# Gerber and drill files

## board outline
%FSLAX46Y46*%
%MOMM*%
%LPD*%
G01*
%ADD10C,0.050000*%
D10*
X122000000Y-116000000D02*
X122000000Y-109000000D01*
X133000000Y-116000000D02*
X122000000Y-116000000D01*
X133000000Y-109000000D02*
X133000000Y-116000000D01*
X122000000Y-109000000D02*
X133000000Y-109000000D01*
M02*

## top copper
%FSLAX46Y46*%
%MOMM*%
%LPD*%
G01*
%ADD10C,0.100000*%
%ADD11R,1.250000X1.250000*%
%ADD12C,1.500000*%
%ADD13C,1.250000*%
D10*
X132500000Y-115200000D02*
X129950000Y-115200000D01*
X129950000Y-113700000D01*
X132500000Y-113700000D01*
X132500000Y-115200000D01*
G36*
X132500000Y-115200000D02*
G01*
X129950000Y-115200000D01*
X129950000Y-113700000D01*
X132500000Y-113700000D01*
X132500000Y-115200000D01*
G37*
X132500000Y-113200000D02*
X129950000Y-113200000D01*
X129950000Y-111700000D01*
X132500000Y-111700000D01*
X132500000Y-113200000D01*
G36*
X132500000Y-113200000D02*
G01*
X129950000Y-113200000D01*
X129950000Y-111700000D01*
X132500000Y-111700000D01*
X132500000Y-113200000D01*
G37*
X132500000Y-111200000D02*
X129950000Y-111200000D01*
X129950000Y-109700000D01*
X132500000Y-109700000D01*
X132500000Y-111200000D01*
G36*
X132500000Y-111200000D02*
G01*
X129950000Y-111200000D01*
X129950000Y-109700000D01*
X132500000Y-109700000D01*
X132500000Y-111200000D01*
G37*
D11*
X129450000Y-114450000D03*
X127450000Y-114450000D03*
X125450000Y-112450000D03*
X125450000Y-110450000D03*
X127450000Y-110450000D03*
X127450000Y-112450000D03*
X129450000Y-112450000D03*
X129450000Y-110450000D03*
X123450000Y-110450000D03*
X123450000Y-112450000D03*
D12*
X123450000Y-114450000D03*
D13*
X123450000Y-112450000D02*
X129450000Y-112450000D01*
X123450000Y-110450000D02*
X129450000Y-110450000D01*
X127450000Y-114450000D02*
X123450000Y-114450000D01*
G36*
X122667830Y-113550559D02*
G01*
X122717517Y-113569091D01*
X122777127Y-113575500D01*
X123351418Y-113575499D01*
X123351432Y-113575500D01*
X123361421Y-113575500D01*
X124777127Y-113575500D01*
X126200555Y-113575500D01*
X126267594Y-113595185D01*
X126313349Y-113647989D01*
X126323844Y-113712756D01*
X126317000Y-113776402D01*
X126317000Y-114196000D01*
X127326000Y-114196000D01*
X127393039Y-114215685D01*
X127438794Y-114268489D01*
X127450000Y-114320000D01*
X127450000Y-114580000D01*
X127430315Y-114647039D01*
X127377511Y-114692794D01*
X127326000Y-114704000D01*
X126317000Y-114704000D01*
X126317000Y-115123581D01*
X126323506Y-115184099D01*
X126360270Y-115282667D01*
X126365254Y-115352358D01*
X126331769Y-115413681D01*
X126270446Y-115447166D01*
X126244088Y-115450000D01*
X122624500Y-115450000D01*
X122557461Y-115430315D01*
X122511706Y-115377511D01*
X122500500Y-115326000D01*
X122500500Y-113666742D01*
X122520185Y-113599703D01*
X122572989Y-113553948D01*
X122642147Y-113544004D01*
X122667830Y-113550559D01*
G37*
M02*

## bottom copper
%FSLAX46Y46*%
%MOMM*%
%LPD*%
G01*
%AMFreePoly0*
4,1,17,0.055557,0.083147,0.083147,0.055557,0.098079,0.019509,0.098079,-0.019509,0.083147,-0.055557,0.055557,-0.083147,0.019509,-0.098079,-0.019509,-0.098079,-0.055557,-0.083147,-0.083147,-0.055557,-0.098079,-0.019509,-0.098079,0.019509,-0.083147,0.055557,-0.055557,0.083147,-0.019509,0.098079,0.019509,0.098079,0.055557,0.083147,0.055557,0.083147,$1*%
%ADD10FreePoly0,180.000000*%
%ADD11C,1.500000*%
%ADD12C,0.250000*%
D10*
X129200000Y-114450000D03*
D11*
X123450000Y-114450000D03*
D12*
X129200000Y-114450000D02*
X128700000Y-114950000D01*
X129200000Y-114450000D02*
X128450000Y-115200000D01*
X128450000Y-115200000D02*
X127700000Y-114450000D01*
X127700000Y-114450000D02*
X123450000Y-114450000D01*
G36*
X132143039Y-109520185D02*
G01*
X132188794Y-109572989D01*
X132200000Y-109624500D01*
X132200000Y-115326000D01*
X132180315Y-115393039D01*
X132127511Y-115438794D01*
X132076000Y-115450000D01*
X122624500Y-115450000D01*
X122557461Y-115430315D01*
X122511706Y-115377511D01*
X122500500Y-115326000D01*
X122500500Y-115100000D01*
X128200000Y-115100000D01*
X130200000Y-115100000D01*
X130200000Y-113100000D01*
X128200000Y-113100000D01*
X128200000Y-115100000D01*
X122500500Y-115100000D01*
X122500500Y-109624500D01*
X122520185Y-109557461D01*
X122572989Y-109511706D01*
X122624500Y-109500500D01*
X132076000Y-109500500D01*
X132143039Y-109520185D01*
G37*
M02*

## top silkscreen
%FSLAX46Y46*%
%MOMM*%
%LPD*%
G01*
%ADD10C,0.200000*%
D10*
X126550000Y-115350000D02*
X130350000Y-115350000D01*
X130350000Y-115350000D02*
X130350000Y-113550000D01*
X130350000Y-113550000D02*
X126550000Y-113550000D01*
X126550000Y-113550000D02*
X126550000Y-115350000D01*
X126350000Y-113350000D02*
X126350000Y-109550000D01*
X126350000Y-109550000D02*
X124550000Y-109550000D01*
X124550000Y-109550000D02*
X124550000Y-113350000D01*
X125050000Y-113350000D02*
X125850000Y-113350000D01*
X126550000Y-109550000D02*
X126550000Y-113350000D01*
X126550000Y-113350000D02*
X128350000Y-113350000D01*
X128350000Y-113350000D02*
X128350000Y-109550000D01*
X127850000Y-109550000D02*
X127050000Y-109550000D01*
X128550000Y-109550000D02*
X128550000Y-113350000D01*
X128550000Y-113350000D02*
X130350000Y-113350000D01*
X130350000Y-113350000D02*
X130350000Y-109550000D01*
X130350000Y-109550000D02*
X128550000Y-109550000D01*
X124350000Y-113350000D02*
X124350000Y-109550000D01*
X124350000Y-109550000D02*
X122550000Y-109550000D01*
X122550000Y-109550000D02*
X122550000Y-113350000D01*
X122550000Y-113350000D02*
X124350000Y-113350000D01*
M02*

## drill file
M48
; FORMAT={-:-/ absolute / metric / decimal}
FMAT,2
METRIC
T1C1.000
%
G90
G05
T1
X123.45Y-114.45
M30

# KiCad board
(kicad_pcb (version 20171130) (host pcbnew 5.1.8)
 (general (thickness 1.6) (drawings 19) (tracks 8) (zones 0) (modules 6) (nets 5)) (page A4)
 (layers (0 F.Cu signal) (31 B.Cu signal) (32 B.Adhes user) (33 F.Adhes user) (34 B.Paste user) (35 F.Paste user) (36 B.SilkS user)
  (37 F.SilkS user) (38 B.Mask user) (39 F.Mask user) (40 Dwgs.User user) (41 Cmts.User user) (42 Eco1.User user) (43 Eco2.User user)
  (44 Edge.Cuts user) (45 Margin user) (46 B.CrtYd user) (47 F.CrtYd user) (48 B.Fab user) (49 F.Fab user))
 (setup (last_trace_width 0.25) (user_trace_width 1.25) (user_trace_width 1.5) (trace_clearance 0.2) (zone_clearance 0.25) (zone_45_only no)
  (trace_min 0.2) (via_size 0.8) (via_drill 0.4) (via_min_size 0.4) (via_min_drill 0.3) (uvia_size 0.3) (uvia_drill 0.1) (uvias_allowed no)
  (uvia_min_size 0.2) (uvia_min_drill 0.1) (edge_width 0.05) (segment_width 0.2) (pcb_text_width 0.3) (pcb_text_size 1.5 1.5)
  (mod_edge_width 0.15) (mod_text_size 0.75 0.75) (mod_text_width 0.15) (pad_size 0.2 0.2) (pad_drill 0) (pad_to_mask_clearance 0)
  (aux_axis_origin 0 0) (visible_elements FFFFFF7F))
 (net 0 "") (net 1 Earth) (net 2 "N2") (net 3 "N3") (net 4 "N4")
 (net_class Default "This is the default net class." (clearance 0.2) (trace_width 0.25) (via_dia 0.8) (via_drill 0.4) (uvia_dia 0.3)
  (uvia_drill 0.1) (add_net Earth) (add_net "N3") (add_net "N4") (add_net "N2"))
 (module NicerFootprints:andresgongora (layer B.Cu) (at 129.2 114.45 180)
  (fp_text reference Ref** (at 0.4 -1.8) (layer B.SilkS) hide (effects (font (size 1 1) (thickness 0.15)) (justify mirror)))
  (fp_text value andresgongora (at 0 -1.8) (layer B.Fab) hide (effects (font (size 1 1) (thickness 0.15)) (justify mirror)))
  (pad 0 smd custom (at 0 0 180) (size 0.2 0.2) (layers B.Cu) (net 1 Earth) (zone_connect 2) (options (clearance outline) (anchor circle))
   (primitives)))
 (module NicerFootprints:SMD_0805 (layer F.Cu) (at 128.45 114.45 270)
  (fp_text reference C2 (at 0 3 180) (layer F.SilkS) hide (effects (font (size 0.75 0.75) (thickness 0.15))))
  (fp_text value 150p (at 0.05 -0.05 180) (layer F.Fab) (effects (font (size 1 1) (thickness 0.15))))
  (fp_line (start 0.9 1.9) (end 0.9 -1.9) (layer F.SilkS) (width 0.2))
  (fp_line (start 0.9 -1.9) (end -0.9 -1.9) (layer F.SilkS) (width 0.2))
  (fp_line (start -0.9 -1.9) (end -0.9 1.9) (layer F.SilkS) (width 0.2))
  (fp_line (start -0.9 1.9) (end 0.9 1.9) (layer F.SilkS) (width 0.2))
  (pad 1 smd rect (at 0 -1 180) (size 1.25 1.25) (layers F.Cu F.Paste F.Mask) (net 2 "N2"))
  (pad 2 smd rect (at 0 1 180) (size 1.25 1.25) (layers F.Cu F.Paste F.Mask) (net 1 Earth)))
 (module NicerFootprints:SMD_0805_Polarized (layer F.Cu) (at 125.45 111.45)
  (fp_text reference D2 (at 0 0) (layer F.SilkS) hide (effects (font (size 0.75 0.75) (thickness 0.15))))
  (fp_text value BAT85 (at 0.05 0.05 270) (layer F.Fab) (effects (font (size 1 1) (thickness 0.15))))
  (fp_line (start 0.9 1.9) (end 0.9 -1.9) (layer F.SilkS) (width 0.2))
  (fp_line (start 0.9 -1.9) (end -0.9 -1.9) (layer F.SilkS) (width 0.2))
  (fp_line (start -0.9 -1.9) (end -0.9 1.9) (layer F.SilkS) (width 0.2))
  (fp_line (start -0.4 1.9) (end 0.4 1.9) (layer F.SilkS) (width 0.2))
  (pad 1 smd rect (at 0 1 270) (size 1.25 1.25) (layers F.Cu F.Paste F.Mask) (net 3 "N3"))
  (pad 2 smd rect (at 0 -1 270) (size 1.25 1.25) (layers F.Cu F.Paste F.Mask) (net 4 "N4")))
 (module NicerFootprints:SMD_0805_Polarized (layer F.Cu) (at 127.45 111.45 180)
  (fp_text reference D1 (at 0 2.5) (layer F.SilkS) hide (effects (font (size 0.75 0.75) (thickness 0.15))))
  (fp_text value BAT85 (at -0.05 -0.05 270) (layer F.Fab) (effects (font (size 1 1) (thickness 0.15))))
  (fp_line (start 0.9 1.9) (end 0.9 -1.9) (layer F.SilkS) (width 0.2))
  (fp_line (start 0.9 -1.9) (end -0.9 -1.9) (layer F.SilkS) (width 0.2))
  (fp_line (start -0.9 -1.9) (end -0.9 1.9) (layer F.SilkS) (width 0.2))
  (fp_line (start -0.4 1.9) (end 0.4 1.9) (layer F.SilkS) (width 0.2))
  (pad 1 smd rect (at 0 1 90) (size 1.25 1.25) (layers F.Cu F.Paste F.Mask) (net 4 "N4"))
  (pad 2 smd rect (at 0 -1 90) (size 1.25 1.25) (layers F.Cu F.Paste F.Mask) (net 3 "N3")))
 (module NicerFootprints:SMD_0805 (layer F.Cu) (at 129.45 111.45 180)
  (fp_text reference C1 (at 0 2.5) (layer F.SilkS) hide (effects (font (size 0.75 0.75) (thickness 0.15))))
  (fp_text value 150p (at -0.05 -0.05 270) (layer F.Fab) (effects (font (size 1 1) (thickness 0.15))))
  (fp_line (start 0.9 1.9) (end 0.9 -1.9) (layer F.SilkS) (width 0.2))
  (fp_line (start 0.9 -1.9) (end -0.9 -1.9) (layer F.SilkS) (width 0.2))
  (fp_line (start -0.9 -1.9) (end -0.9 1.9) (layer F.SilkS) (width 0.2))
  (fp_line (start -0.9 1.9) (end 0.9 1.9) (layer F.SilkS) (width 0.2))
  (pad 1 smd rect (at 0 -1 90) (size 1.25 1.25) (layers F.Cu F.Paste F.Mask) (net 3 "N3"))
  (pad 2 smd rect (at 0 1 90) (size 1.25 1.25) (layers F.Cu F.Paste F.Mask) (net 4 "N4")))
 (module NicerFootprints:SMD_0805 (layer F.Cu) (at 123.45 111.45)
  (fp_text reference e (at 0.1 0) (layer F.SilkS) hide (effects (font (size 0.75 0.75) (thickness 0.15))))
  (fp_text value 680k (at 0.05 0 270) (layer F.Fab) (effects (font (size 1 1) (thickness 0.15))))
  (fp_line (start 0.9 1.9) (end 0.9 -1.9) (layer F.SilkS) (width 0.2))
  (fp_line (start 0.9 -1.9) (end -0.9 -1.9) (layer F.SilkS) (width 0.2))
  (fp_line (start -0.9 -1.9) (end -0.9 1.9) (layer F.SilkS) (width 0.2))
  (fp_line (start -0.9 1.9) (end 0.9 1.9) (layer F.SilkS) (width 0.2))
  (pad 1 smd rect (at 0 -1 270) (size 1.25 1.25) (layers F.Cu F.Paste F.Mask) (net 4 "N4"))
  (pad 2 smd rect (at 0 1 270) (size 1.25 1.25) (layers F.Cu F.Paste F.Mask) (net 3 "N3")))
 (gr_line (start 122 116) (end 122 109) (layer Edge.Cuts) (width 0.05))
 (gr_line (start 133 116) (end 122 116) (layer Edge.Cuts) (width 0.05))
 (gr_line (start 133 109) (end 133 116) (layer Edge.Cuts) (width 0.05))
 (gr_line (start 122 109) (end 133 109) (layer Edge.Cuts) (width 0.05))
 (gr_poly (pts (xy 132.5 115.2) (xy 129.95 115.2) (xy 129.95 113.7) (xy 132.5 113.7)) (layer F.Cu) (width 0.1))
 (gr_poly (pts (xy 132.5 113.2) (xy 129.95 113.2) (xy 129.95 111.7) (xy 132.5 111.7)) (layer F.Cu) (width 0.1))
 (gr_poly (pts (xy 132.5 111.2) (xy 129.95 111.2) (xy 129.95 109.7) (xy 132.5 109.7)) (layer F.Cu) (width 0.1))
 (segment (start 123.45 112.45) (end 129.45 112.45) (width 1.25) (layer F.Cu) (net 3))
 (segment (start 123.45 110.45) (end 129.45 110.45) (width 1.25) (layer F.Cu) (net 4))
 (via (at 123.45 114.45) (size 1.5) (drill 1) (layers F.Cu B.Cu) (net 1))
 (segment (start 127.45 114.45) (end 123.45 114.45) (width 1.25) (layer F.Cu) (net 1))
 (segment (start 129.2 114.45) (end 128.7 114.95) (width 0.25) (layer B.Cu) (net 1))
 (segment (start 129.2 114.45) (end 128.45 115.2) (width 0.25) (layer B.Cu) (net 1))
 (segment (start 128.45 115.2) (end 127.7 114.45) (width 0.25) (layer B.Cu) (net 1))
 (segment (start 127.7 114.45) (end 123.45 114.45) (width 0.25) (layer B.Cu) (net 1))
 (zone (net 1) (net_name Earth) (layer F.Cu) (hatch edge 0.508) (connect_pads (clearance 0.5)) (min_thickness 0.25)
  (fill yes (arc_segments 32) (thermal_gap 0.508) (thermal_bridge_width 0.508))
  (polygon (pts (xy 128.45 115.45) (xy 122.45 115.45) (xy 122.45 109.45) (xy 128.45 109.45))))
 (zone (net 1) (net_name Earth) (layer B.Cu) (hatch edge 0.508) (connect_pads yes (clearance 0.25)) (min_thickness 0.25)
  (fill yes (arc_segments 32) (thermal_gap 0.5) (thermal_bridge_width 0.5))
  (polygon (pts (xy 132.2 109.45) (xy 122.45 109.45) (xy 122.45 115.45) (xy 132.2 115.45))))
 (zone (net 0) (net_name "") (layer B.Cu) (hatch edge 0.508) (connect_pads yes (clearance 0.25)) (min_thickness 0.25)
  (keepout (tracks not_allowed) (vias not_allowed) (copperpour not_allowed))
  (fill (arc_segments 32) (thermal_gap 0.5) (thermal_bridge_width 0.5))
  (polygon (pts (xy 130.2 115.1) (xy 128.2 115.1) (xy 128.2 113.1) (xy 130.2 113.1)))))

